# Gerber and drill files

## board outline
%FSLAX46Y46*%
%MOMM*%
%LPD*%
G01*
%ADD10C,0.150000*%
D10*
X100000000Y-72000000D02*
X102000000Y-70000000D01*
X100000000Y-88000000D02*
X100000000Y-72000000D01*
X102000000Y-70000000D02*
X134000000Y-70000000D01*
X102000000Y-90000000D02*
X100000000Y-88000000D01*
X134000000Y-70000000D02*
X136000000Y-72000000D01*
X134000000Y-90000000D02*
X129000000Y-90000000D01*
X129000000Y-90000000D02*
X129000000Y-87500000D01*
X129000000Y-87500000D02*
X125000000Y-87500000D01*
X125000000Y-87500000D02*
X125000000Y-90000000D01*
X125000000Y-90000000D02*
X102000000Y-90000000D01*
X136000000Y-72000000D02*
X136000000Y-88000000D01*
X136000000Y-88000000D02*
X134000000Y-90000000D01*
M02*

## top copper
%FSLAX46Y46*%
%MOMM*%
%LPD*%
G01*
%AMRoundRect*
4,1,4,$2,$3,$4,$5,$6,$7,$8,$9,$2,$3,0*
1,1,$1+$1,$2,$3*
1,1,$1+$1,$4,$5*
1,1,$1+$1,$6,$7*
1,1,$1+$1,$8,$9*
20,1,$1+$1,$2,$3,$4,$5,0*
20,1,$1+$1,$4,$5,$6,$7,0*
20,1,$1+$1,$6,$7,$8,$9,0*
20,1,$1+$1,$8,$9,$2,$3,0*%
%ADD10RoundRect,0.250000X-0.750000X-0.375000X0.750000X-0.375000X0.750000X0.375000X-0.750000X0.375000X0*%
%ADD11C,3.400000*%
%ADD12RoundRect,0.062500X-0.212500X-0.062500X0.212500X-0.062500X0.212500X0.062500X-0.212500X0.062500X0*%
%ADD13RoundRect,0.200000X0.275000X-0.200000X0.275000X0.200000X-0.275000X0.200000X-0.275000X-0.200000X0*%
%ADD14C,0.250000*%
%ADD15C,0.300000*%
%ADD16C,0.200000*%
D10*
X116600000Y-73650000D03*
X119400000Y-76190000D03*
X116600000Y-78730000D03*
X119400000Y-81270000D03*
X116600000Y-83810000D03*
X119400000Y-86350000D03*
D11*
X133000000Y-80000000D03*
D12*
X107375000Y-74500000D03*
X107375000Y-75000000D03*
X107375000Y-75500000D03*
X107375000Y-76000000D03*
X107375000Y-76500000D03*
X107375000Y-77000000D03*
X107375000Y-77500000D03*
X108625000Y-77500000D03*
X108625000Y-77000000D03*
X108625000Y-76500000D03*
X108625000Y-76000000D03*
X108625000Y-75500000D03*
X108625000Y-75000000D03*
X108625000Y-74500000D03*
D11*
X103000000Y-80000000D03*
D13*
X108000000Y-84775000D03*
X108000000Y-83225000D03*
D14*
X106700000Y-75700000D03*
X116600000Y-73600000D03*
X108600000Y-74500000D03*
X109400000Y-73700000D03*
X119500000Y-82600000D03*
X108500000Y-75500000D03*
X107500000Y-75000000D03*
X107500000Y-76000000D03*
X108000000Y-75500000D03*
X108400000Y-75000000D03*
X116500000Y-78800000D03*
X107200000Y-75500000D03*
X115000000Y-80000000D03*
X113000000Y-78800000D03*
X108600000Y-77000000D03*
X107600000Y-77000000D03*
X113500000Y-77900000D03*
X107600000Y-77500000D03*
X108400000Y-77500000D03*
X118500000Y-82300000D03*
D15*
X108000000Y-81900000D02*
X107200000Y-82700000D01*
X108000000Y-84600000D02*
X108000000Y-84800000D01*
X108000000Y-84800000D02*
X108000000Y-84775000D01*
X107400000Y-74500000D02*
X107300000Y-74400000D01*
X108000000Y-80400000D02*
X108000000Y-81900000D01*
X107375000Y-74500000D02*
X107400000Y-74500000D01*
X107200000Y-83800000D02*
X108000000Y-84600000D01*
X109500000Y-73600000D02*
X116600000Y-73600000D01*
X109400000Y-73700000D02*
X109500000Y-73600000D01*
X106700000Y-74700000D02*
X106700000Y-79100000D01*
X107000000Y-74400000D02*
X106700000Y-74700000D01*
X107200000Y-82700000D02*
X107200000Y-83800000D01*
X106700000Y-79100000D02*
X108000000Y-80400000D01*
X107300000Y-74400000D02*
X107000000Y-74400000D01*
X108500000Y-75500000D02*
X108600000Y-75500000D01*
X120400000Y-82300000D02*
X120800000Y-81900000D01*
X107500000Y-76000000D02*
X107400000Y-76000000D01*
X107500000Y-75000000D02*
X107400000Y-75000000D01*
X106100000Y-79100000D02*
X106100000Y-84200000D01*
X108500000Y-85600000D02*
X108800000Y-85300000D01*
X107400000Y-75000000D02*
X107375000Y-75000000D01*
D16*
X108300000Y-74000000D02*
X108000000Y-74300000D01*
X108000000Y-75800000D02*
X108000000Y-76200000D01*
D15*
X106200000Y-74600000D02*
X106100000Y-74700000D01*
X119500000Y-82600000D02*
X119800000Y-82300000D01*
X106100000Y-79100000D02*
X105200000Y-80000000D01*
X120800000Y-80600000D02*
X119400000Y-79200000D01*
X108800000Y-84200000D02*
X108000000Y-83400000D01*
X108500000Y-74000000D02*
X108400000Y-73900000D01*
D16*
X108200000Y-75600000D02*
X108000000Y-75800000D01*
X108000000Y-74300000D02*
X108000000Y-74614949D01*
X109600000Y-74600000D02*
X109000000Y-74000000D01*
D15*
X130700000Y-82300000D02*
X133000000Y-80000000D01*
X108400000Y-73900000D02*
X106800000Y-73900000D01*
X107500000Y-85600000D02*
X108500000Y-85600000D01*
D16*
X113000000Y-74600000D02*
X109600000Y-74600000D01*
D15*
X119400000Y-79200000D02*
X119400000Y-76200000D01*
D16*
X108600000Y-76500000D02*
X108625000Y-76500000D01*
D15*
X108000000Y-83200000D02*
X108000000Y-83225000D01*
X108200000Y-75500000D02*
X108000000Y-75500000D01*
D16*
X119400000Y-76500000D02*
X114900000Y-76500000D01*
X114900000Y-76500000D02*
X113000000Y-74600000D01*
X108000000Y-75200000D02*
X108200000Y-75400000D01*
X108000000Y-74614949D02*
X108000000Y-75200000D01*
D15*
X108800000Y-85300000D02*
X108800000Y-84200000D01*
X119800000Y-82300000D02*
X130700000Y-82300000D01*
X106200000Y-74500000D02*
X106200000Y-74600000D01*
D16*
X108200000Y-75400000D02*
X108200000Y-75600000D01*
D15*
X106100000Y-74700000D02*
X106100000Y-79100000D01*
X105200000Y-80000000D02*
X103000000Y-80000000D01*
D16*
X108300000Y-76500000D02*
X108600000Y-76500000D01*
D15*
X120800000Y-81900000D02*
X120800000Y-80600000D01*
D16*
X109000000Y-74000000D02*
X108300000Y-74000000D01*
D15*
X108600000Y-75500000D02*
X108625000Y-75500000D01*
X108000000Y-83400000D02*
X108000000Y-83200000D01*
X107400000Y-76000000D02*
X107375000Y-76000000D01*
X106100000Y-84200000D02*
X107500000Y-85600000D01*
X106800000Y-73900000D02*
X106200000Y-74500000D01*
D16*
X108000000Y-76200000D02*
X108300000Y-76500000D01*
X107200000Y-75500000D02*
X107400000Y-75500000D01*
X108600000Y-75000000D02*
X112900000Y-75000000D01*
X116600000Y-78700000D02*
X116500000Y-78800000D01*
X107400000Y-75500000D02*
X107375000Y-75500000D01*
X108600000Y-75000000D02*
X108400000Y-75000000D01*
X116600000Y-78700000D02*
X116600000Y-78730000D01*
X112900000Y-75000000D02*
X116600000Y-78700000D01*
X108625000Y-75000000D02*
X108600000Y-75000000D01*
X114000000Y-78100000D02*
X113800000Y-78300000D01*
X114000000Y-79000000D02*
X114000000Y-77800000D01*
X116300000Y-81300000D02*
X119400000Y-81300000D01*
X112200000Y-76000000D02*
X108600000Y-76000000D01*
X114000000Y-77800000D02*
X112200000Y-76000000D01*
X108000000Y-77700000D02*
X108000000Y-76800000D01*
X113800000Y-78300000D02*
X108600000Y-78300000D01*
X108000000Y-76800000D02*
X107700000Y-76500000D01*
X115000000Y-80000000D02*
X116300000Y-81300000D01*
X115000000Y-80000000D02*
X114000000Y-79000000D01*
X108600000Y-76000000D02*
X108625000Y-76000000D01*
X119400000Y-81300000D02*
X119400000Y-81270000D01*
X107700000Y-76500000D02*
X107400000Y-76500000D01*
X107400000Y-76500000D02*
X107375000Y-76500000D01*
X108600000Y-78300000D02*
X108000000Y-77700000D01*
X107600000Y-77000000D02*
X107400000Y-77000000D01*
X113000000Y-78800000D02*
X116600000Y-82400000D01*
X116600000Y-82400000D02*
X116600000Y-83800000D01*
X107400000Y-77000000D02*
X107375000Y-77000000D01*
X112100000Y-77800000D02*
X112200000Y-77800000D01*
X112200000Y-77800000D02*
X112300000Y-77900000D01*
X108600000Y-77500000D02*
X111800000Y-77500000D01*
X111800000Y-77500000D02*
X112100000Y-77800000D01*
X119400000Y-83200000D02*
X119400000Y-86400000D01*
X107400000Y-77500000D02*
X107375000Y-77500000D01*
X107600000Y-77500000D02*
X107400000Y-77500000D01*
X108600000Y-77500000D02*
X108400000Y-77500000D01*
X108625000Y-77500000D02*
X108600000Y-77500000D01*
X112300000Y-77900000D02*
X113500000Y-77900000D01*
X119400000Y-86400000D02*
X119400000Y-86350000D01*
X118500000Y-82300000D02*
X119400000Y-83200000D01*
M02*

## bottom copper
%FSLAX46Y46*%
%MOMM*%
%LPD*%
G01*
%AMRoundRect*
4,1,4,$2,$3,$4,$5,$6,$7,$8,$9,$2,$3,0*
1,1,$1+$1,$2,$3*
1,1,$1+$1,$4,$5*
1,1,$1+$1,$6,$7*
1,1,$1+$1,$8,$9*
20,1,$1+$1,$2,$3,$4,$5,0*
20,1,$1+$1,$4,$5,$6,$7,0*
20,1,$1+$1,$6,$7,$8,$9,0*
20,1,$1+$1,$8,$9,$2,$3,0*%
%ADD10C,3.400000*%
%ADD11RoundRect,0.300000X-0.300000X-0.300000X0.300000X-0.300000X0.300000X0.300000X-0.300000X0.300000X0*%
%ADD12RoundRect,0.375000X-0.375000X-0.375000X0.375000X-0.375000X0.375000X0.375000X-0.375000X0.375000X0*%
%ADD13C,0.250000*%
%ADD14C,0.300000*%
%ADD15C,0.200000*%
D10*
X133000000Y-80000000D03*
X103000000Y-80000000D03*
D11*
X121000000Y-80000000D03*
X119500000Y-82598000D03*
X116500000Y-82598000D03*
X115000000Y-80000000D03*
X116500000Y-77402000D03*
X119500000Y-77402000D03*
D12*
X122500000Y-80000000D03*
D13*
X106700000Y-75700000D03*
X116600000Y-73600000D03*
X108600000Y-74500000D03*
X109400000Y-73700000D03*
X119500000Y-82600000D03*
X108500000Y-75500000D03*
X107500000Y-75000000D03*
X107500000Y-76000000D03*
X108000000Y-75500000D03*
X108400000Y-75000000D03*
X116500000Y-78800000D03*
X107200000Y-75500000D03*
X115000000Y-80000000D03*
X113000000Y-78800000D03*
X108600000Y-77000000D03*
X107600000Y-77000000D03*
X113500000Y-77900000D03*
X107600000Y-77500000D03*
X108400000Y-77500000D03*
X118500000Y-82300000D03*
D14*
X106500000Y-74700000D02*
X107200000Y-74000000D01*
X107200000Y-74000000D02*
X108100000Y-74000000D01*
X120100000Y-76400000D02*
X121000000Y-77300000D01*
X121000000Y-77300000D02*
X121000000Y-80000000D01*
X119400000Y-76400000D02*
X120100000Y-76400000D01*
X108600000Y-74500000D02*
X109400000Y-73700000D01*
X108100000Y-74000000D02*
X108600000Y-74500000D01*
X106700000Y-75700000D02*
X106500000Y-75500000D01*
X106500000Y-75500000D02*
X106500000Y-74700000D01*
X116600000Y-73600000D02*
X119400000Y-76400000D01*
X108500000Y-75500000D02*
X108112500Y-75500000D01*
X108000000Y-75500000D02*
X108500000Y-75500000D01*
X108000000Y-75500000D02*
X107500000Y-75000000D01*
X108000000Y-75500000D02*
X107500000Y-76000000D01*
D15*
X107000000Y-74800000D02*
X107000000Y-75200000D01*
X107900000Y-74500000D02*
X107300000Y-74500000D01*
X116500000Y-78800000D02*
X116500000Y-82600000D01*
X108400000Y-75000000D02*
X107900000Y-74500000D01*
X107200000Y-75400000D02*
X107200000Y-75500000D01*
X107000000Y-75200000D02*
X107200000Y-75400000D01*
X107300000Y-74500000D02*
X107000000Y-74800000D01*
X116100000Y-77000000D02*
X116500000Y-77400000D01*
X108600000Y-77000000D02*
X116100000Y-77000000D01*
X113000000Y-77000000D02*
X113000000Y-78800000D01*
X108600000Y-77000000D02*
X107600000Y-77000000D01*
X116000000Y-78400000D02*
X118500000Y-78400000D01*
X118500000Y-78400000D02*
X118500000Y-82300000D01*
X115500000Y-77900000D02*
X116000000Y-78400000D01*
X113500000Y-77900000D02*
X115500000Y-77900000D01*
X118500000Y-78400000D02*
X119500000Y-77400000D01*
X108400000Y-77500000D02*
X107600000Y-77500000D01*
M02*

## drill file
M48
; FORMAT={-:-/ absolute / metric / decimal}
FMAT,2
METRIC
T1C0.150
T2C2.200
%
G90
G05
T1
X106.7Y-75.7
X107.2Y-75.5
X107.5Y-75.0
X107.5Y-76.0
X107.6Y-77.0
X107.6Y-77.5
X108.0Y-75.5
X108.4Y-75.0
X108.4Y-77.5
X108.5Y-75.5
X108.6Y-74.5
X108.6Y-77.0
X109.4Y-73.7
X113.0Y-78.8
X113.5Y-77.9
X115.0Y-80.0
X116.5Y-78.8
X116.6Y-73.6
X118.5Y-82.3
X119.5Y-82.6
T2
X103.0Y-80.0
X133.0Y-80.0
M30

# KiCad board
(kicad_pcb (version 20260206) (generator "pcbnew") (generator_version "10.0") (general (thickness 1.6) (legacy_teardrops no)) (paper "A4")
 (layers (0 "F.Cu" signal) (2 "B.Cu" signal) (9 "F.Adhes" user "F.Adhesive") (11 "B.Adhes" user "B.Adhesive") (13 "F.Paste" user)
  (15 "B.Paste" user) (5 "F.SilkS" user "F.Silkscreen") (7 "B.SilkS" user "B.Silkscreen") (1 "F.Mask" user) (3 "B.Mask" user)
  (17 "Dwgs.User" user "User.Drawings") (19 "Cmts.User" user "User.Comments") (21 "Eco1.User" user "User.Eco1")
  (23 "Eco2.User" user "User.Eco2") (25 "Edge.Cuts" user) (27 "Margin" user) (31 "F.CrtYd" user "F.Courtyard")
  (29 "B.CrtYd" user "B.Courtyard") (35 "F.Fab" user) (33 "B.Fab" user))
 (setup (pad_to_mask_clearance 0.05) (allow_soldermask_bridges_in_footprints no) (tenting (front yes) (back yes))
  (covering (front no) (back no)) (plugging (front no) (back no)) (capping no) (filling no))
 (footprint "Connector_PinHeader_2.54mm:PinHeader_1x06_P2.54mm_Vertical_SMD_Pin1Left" (layer "F.Cu") (at 118 73.65)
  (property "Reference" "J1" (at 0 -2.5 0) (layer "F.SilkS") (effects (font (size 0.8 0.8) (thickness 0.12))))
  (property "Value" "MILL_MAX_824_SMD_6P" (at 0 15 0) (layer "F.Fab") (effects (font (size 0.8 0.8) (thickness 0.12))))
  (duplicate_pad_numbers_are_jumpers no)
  (pad "1" smd roundrect (at -1.4 0) (size 2 1.25) (layers "F.Cu" "F.Mask" "F.Paste") (roundrect_rratio 0.2) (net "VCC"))
  (pad "2" smd roundrect (at 1.4 2.54) (size 2 1.25) (layers "F.Cu" "F.Mask" "F.Paste") (roundrect_rratio 0.2) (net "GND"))
  (pad "3" smd roundrect (at -1.4 5.08) (size 2 1.25) (layers "F.Cu" "F.Mask" "F.Paste") (roundrect_rratio 0.2) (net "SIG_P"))
  (pad "4" smd roundrect (at 1.4 7.62) (size 2 1.25) (layers "F.Cu" "F.Mask" "F.Paste") (roundrect_rratio 0.2) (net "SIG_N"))
  (pad "5" smd roundrect (at -1.4 10.16) (size 2 1.25) (layers "F.Cu" "F.Mask" "F.Paste") (roundrect_rratio 0.2) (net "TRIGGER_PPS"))
  (pad "6" smd roundrect (at 1.4 12.7) (size 2 1.25) (layers "F.Cu" "F.Mask" "F.Paste") (roundrect_rratio 0.2) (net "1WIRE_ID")))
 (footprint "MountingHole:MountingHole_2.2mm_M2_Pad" (layer "F.Cu") (at 133 80)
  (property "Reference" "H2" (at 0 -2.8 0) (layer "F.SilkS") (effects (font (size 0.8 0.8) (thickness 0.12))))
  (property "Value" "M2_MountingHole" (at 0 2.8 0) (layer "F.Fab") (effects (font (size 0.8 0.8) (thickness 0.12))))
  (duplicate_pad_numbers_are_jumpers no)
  (pad "1" thru_hole circle (at 0 0) (size 3.4 3.4) (drill 2.2) (layers "*.Cu" "*.Mask") (remove_unused_layers no) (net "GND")))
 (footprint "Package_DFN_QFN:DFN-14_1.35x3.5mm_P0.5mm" (layer "F.Cu") (at 108 76)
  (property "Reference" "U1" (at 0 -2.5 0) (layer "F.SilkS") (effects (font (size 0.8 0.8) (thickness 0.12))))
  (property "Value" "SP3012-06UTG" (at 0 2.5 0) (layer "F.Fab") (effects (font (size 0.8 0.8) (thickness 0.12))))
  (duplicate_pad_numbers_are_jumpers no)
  (pad "1" smd roundrect (at -0.625 -1.5) (size 0.55 0.25) (layers "F.Cu" "F.Mask" "F.Paste") (roundrect_rratio 0.25) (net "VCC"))
  (pad "2" smd roundrect (at -0.625 -1) (size 0.55 0.25) (layers "F.Cu" "F.Mask" "F.Paste") (roundrect_rratio 0.25) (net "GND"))
  (pad "3" smd roundrect (at -0.625 -0.5) (size 0.55 0.25) (layers "F.Cu" "F.Mask" "F.Paste") (roundrect_rratio 0.25) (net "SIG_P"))
  (pad "4" smd roundrect (at -0.625 0) (size 0.55 0.25) (layers "F.Cu" "F.Mask" "F.Paste") (roundrect_rratio 0.25) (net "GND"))
  (pad "5" smd roundrect (at -0.625 0.5) (size 0.55 0.25) (layers "F.Cu" "F.Mask" "F.Paste") (roundrect_rratio 0.25) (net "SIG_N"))
  (pad "6" smd roundrect (at -0.625 1) (size 0.55 0.25) (layers "F.Cu" "F.Mask" "F.Paste") (roundrect_rratio 0.25) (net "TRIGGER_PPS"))
  (pad "7" smd roundrect (at -0.625 1.5) (size 0.55 0.25) (layers "F.Cu" "F.Mask" "F.Paste") (roundrect_rratio 0.25) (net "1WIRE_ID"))
  (pad "8" smd roundrect (at 0.625 1.5) (size 0.55 0.25) (layers "F.Cu" "F.Mask" "F.Paste") (roundrect_rratio 0.25) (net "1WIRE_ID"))
  (pad "9" smd roundrect (at 0.625 1) (size 0.55 0.25) (layers "F.Cu" "F.Mask" "F.Paste") (roundrect_rratio 0.25) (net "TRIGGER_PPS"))
  (pad "10" smd roundrect (at 0.625 0.5) (size 0.55 0.25) (layers "F.Cu" "F.Mask" "F.Paste") (roundrect_rratio 0.25) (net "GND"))
  (pad "11" smd roundrect (at 0.625 0) (size 0.55 0.25) (layers "F.Cu" "F.Mask" "F.Paste") (roundrect_rratio 0.25) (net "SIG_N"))
  (pad "12" smd roundrect (at 0.625 -0.5) (size 0.55 0.25) (layers "F.Cu" "F.Mask" "F.Paste") (roundrect_rratio 0.25) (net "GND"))
  (pad "13" smd roundrect (at 0.625 -1) (size 0.55 0.25) (layers "F.Cu" "F.Mask" "F.Paste") (roundrect_rratio 0.25) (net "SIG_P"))
  (pad "14" smd roundrect (at 0.625 -1.5) (size 0.55 0.25) (layers "F.Cu" "F.Mask" "F.Paste") (roundrect_rratio 0.25) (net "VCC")))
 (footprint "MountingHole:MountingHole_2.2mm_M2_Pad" (layer "F.Cu") (at 103 80)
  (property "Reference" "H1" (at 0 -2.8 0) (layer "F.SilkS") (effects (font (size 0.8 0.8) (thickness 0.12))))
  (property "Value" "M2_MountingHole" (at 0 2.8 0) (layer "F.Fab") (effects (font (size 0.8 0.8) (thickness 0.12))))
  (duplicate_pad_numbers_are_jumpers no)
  (pad "1" thru_hole circle (at 0 0) (size 3.4 3.4) (drill 2.2) (layers "*.Cu" "*.Mask") (remove_unused_layers no) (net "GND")))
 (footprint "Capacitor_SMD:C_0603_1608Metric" (layer "F.Cu") (at 108 84 90)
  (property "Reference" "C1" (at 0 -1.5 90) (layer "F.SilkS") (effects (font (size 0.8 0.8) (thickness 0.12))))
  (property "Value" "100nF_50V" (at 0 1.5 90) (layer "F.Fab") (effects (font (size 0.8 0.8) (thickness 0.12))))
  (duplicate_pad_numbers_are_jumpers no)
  (pad "1" smd roundrect (at -0.775 0 90) (size 0.8 0.95) (layers "F.Cu" "F.Mask" "F.Paste") (roundrect_rratio 0.25) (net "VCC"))
  (pad "2" smd roundrect (at 0.775 0 90) (size 0.8 0.95) (layers "F.Cu" "F.Mask" "F.Paste") (roundrect_rratio 0.25) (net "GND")))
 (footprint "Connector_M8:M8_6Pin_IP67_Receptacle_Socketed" (layer "B.Cu") (at 118 80)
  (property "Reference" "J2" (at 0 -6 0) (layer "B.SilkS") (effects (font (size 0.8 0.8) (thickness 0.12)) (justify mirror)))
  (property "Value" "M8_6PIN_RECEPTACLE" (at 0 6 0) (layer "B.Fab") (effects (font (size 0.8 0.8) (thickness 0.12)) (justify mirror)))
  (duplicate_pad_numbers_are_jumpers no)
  (pad "1" smd roundrect (at 3 0) (size 1.2 1.2) (layers "B.Cu" "B.Mask" "B.Paste") (roundrect_rratio 0.25) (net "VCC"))
  (pad "2" smd roundrect (at 1.5 2.598) (size 1.2 1.2) (layers "B.Cu" "B.Mask" "B.Paste") (roundrect_rratio 0.25) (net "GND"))
  (pad "3" smd roundrect (at -1.5 2.598) (size 1.2 1.2) (layers "B.Cu" "B.Mask" "B.Paste") (roundrect_rratio 0.25) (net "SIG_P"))
  (pad "4" smd roundrect (at -3 0) (size 1.2 1.2) (layers "B.Cu" "B.Mask" "B.Paste") (roundrect_rratio 0.25) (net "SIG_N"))
  (pad "5" smd roundrect (at -1.5 -2.598) (size 1.2 1.2) (layers "B.Cu" "B.Mask" "B.Paste") (roundrect_rratio 0.25) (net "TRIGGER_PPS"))
  (pad "6" smd roundrect (at 1.5 -2.598) (size 1.2 1.2) (layers "B.Cu" "B.Mask" "B.Paste") (roundrect_rratio 0.25) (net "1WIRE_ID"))
  (pad "7" smd roundrect (at 4.5 0) (size 1.5 1.5) (layers "B.Cu" "B.Mask" "B.Paste") (roundrect_rratio 0.25) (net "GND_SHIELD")))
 (gr_line (start 100 72) (end 102 70) (stroke (width 0.15) (type solid)) (layer "Edge.Cuts"))
 (gr_line (start 100 88) (end 100 72) (stroke (width 0.15) (type solid)) (layer "Edge.Cuts"))
 (gr_line (start 102 70) (end 134 70) (stroke (width 0.15) (type solid)) (layer "Edge.Cuts"))
 (gr_line (start 102 90) (end 100 88) (stroke (width 0.15) (type solid)) (layer "Edge.Cuts"))
 (gr_line (start 134 70) (end 136 72) (stroke (width 0.15) (type solid)) (layer "Edge.Cuts"))
 (gr_line (start 134 90) (end 129 90) (stroke (width 0.15) (type solid)) (layer "Edge.Cuts"))
 (gr_line (start 129 90) (end 129 87.5) (stroke (width 0.15) (type solid)) (layer "Edge.Cuts"))
 (gr_line (start 129 87.5) (end 125 87.5) (stroke (width 0.15) (type solid)) (layer "Edge.Cuts"))
 (gr_line (start 125 87.5) (end 125 90) (stroke (width 0.15) (type solid)) (layer "Edge.Cuts"))
 (gr_line (start 125 90) (end 102 90) (stroke (width 0.15) (type solid)) (layer "Edge.Cuts"))
 (gr_line (start 136 72) (end 136 88) (stroke (width 0.15) (type solid)) (layer "Edge.Cuts"))
 (gr_line (start 136 88) (end 134 90) (stroke (width 0.15) (type solid)) (layer "Edge.Cuts"))
 (segment (start 108 81.9) (end 107.2 82.7) (width 0.3) (layer "F.Cu") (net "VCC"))
 (segment (start 108 84.6) (end 108 84.8) (width 0.3) (layer "F.Cu") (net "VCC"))
 (segment (start 108 84.8) (end 108 84.775) (width 0.3) (layer "F.Cu") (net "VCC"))
 (segment (start 107.4 74.5) (end 107.3 74.4) (width 0.3) (layer "F.Cu") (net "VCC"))
 (segment (start 108 80.4) (end 108 81.9) (width 0.3) (layer "F.Cu") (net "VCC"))
 (segment (start 107.375 74.5) (end 107.4 74.5) (width 0.3) (layer "F.Cu") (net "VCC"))
 (segment (start 107.2 83.8) (end 108 84.6) (width 0.3) (layer "F.Cu") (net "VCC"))
 (segment (start 109.5 73.6) (end 116.6 73.6) (width 0.3) (layer "F.Cu") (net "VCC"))
 (segment (start 109.4 73.7) (end 109.5 73.6) (width 0.3) (layer "F.Cu") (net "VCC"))
 (segment (start 106.7 74.7) (end 106.7 79.1) (width 0.3) (layer "F.Cu") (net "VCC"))
 (segment (start 107 74.4) (end 106.7 74.7) (width 0.3) (layer "F.Cu") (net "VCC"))
 (segment (start 107.2 82.7) (end 107.2 83.8) (width 0.3) (layer "F.Cu") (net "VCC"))
 (segment (start 106.7 79.1) (end 108 80.4) (width 0.3) (layer "F.Cu") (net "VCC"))
 (segment (start 107.3 74.4) (end 107 74.4) (width 0.3) (layer "F.Cu") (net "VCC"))
 (via (at 106.7 75.7) (size 0.25) (drill 0.15) (layers "F.Cu" "B.Cu") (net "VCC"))
 (via (at 116.6 73.6) (size 0.25) (drill 0.15) (layers "F.Cu" "B.Cu") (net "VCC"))
 (via (at 108.6 74.5) (size 0.25) (drill 0.15) (layers "F.Cu" "B.Cu") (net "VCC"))
 (via (at 109.4 73.7) (size 0.25) (drill 0.15) (layers "F.Cu" "B.Cu") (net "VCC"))
 (segment (start 106.5 74.7) (end 107.2 74) (width 0.3) (layer "B.Cu") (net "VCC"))
 (segment (start 107.2 74) (end 108.1 74) (width 0.3) (layer "B.Cu") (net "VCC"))
 (segment (start 120.1 76.4) (end 121 77.3) (width 0.3) (layer "B.Cu") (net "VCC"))
 (segment (start 121 77.3) (end 121 80) (width 0.3) (layer "B.Cu") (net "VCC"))
 (segment (start 119.4 76.4) (end 120.1 76.4) (width 0.3) (layer "B.Cu") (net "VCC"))
 (segment (start 108.6 74.5) (end 109.4 73.7) (width 0.3) (layer "B.Cu") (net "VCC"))
 (segment (start 108.1 74) (end 108.6 74.5) (width 0.3) (layer "B.Cu") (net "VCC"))
 (segment (start 106.7 75.7) (end 106.5 75.5) (width 0.3) (layer "B.Cu") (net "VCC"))
 (segment (start 106.5 75.5) (end 106.5 74.7) (width 0.3) (layer "B.Cu") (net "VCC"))
 (segment (start 116.6 73.6) (end 119.4 76.4) (width 0.3) (layer "B.Cu") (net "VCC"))
 (segment (start 108.5 75.5) (end 108.6 75.5) (width 0.3) (layer "F.Cu") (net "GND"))
 (segment (start 120.4 82.3) (end 120.8 81.9) (width 0.3) (layer "F.Cu") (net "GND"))
 (segment (start 107.5 76) (end 107.4 76) (width 0.3) (layer "F.Cu") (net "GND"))
 (segment (start 107.5 75) (end 107.4 75) (width 0.3) (layer "F.Cu") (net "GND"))
 (segment (start 106.1 79.1) (end 106.1 84.2) (width 0.3) (layer "F.Cu") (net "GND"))
 (segment (start 108.5 85.6) (end 108.8 85.3) (width 0.3) (layer "F.Cu") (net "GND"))
 (segment (start 107.4 75) (end 107.375 75) (width 0.3) (layer "F.Cu") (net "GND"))
 (segment (start 108.3 74) (end 108 74.3) (width 0.2) (layer "F.Cu") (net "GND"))
 (segment (start 108 75.8) (end 108 76.2) (width 0.2) (layer "F.Cu") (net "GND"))
 (segment (start 106.2 74.6) (end 106.1 74.7) (width 0.3) (layer "F.Cu") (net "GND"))
 (segment (start 119.5 82.6) (end 119.8 82.3) (width 0.3) (layer "F.Cu") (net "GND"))
 (segment (start 106.1 79.1) (end 105.2 80) (width 0.3) (layer "F.Cu") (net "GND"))
 (segment (start 120.8 80.6) (end 119.4 79.2) (width 0.3) (layer "F.Cu") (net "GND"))
 (segment (start 108.8 84.2) (end 108 83.4) (width 0.3) (layer "F.Cu") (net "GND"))
 (segment (start 108.5 74) (end 108.4 73.9) (width 0.3) (layer "F.Cu") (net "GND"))
 (segment (start 108.2 75.6) (end 108 75.8) (width 0.2) (layer "F.Cu") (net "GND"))
 (segment (start 108 74.3) (end 108 74.614949) (width 0.2) (layer "F.Cu") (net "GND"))
 (segment (start 109.6 74.6) (end 109 74) (width 0.2) (layer "F.Cu") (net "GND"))
 (segment (start 130.7 82.3) (end 133 80) (width 0.3) (layer "F.Cu") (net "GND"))
 (segment (start 108.4 73.9) (end 106.8 73.9) (width 0.3) (layer "F.Cu") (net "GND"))
 (segment (start 107.5 85.6) (end 108.5 85.6) (width 0.3) (layer "F.Cu") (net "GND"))
 (segment (start 113 74.6) (end 109.6 74.6) (width 0.2) (layer "F.Cu") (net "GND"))
 (segment (start 119.4 79.2) (end 119.4 76.2) (width 0.3) (layer "F.Cu") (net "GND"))
 (segment (start 108.6 76.5) (end 108.625 76.5) (width 0.2) (layer "F.Cu") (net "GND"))
 (segment (start 108 83.2) (end 108 83.225) (width 0.3) (layer "F.Cu") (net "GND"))
 (segment (start 108.2 75.5) (end 108 75.5) (width 0.3) (layer "F.Cu") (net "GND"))
 (segment (start 119.4 76.5) (end 114.9 76.5) (width 0.2) (layer "F.Cu") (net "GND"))
 (segment (start 114.9 76.5) (end 113 74.6) (width 0.2) (layer "F.Cu") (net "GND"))
 (segment (start 108 75.2) (end 108.2 75.4) (width 0.2) (layer "F.Cu") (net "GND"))
 (segment (start 108 74.614949) (end 108 75.2) (width 0.2) (layer "F.Cu") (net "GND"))
 (segment (start 108.8 85.3) (end 108.8 84.2) (width 0.3) (layer "F.Cu") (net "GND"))
 (segment (start 119.8 82.3) (end 130.7 82.3) (width 0.3) (layer "F.Cu") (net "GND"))
 (segment (start 106.2 74.5) (end 106.2 74.6) (width 0.3) (layer "F.Cu") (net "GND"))
 (segment (start 108.2 75.4) (end 108.2 75.6) (width 0.2) (layer "F.Cu") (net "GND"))
 (segment (start 106.1 74.7) (end 106.1 79.1) (width 0.3) (layer "F.Cu") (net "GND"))
 (segment (start 105.2 80) (end 103 80) (width 0.3) (layer "F.Cu") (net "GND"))
 (segment (start 108.3 76.5) (end 108.6 76.5) (width 0.2) (layer "F.Cu") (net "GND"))
 (segment (start 120.8 81.9) (end 120.8 80.6) (width 0.3) (layer "F.Cu") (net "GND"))
 (segment (start 109 74) (end 108.3 74) (width 0.2) (layer "F.Cu") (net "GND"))
 (segment (start 108.6 75.5) (end 108.625 75.5) (width 0.3) (layer "F.Cu") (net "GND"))
 (segment (start 108 83.4) (end 108 83.2) (width 0.3) (layer "F.Cu") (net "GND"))
 (segment (start 107.4 76) (end 107.375 76) (width 0.3) (layer "F.Cu") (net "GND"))
 (segment (start 106.1 84.2) (end 107.5 85.6) (width 0.3) (layer "F.Cu") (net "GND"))
 (segment (start 106.8 73.9) (end 106.2 74.5) (width 0.3) (layer "F.Cu") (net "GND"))
 (segment (start 108 76.2) (end 108.3 76.5) (width 0.2) (layer "F.Cu") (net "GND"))
 (via (at 119.5 82.6) (size 0.25) (drill 0.15) (layers "F.Cu" "B.Cu") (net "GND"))
 (via (at 108.5 75.5) (size 0.25) (drill 0.15) (layers "F.Cu" "B.Cu") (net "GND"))
 (via (at 107.5 75) (size 0.25) (drill 0.15) (layers "F.Cu" "B.Cu") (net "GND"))
 (via (at 107.5 76) (size 0.25) (drill 0.15) (layers "F.Cu" "B.Cu") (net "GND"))
 (via (at 108 75.5) (size 0.25) (drill 0.15) (layers "F.Cu" "B.Cu") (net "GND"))
 (segment (start 108.5 75.5) (end 108.1125 75.5) (width 0.3) (layer "B.Cu") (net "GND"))
 (segment (start 108 75.5) (end 108.5 75.5) (width 0.3) (layer "B.Cu") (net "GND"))
 (segment (start 108 75.5) (end 107.5 75) (width 0.3) (layer "B.Cu") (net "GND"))
 (segment (start 108 75.5) (end 107.5 76) (width 0.3) (layer "B.Cu") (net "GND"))
 (segment (start 107.2 75.5) (end 107.4 75.5) (width 0.2) (layer "F.Cu") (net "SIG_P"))
 (segment (start 108.6 75) (end 112.9 75) (width 0.2) (layer "F.Cu") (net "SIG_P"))
 (segment (start 116.6 78.7) (end 116.5 78.8) (width 0.2) (layer "F.Cu") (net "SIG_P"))
 (segment (start 107.4 75.5) (end 107.375 75.5) (width 0.2) (layer "F.Cu") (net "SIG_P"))
 (segment (start 108.6 75) (end 108.4 75) (width 0.2) (layer "F.Cu") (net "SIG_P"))
 (segment (start 116.6 78.7) (end 116.6 78.73) (width 0.2) (layer "F.Cu") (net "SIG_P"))
 (segment (start 112.9 75) (end 116.6 78.7) (width 0.2) (layer "F.Cu") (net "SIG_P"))
 (segment (start 108.625 75) (end 108.6 75) (width 0.2) (layer "F.Cu") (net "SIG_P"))
 (via (at 108.4 75) (size 0.25) (drill 0.15) (layers "F.Cu" "B.Cu") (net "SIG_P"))
 (via (at 116.5 78.8) (size 0.25) (drill 0.15) (layers "F.Cu" "B.Cu") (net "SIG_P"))
 (via (at 107.2 75.5) (size 0.25) (drill 0.15) (layers "F.Cu" "B.Cu") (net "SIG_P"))
 (segment (start 107 74.8) (end 107 75.2) (width 0.2) (layer "B.Cu") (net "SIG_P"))
 (segment (start 107.9 74.5) (end 107.3 74.5) (width 0.2) (layer "B.Cu") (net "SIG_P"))
 (segment (start 116.5 78.8) (end 116.5 82.6) (width 0.2) (layer "B.Cu") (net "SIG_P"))
 (segment (start 108.4 75) (end 107.9 74.5) (width 0.2) (layer "B.Cu") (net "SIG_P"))
 (segment (start 107.2 75.4) (end 107.2 75.5) (width 0.2) (layer "B.Cu") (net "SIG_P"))
 (segment (start 107 75.2) (end 107.2 75.4) (width 0.2) (layer "B.Cu") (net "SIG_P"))
 (segment (start 107.3 74.5) (end 107 74.8) (width 0.2) (layer "B.Cu") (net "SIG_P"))
 (segment (start 114 78.1) (end 113.8 78.3) (width 0.2) (layer "F.Cu") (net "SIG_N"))
 (segment (start 114 79) (end 114 77.8) (width 0.2) (layer "F.Cu") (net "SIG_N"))
 (segment (start 116.3 81.3) (end 119.4 81.3) (width 0.2) (layer "F.Cu") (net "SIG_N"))
 (segment (start 112.2 76) (end 108.6 76) (width 0.2) (layer "F.Cu") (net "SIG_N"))
 (segment (start 114 77.8) (end 112.2 76) (width 0.2) (layer "F.Cu") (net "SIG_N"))
 (segment (start 108 77.7) (end 108 76.8) (width 0.2) (layer "F.Cu") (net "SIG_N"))
 (segment (start 113.8 78.3) (end 108.6 78.3) (width 0.2) (layer "F.Cu") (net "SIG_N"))
 (segment (start 108 76.8) (end 107.7 76.5) (width 0.2) (layer "F.Cu") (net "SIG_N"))
 (segment (start 115 80) (end 116.3 81.3) (width 0.2) (layer "F.Cu") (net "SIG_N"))
 (segment (start 115 80) (end 114 79) (width 0.2) (layer "F.Cu") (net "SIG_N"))
 (segment (start 108.6 76) (end 108.625 76) (width 0.2) (layer "F.Cu") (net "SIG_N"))
 (segment (start 119.4 81.3) (end 119.4 81.27) (width 0.2) (layer "F.Cu") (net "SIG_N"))
 (segment (start 107.7 76.5) (end 107.4 76.5) (width 0.2) (layer "F.Cu") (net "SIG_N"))
 (segment (start 107.4 76.5) (end 107.375 76.5) (width 0.2) (layer "F.Cu") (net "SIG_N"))
 (segment (start 108.6 78.3) (end 108 77.7) (width 0.2) (layer "F.Cu") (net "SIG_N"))
 (via (at 115 80) (size 0.25) (drill 0.15) (layers "F.Cu" "B.Cu") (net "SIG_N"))
 (segment (start 107.6 77) (end 107.4 77) (width 0.2) (layer "F.Cu") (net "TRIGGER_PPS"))
 (segment (start 113 78.8) (end 116.6 82.4) (width 0.2) (layer "F.Cu") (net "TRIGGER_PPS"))
 (segment (start 116.6 82.4) (end 116.6 83.8) (width 0.2) (layer "F.Cu") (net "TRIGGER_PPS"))
 (segment (start 107.4 77) (end 107.375 77) (width 0.2) (layer "F.Cu") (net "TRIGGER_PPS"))
 (via (at 113 78.8) (size 0.25) (drill 0.15) (layers "F.Cu" "B.Cu") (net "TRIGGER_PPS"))
 (via (at 108.6 77) (size 0.25) (drill 0.15) (layers "F.Cu" "B.Cu") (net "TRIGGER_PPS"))
 (via (at 107.6 77) (size 0.25) (drill 0.15) (layers "F.Cu" "B.Cu") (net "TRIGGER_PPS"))
 (segment (start 116.1 77) (end 116.5 77.4) (width 0.2) (layer "B.Cu") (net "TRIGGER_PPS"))
 (segment (start 108.6 77) (end 116.1 77) (width 0.2) (layer "B.Cu") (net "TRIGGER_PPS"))
 (segment (start 113 77) (end 113 78.8) (width 0.2) (layer "B.Cu") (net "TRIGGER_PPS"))
 (segment (start 108.6 77) (end 107.6 77) (width 0.2) (layer "B.Cu") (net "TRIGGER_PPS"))
 (segment (start 112.1 77.8) (end 112.2 77.8) (width 0.2) (layer "F.Cu") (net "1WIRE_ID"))
 (segment (start 112.2 77.8) (end 112.3 77.9) (width 0.2) (layer "F.Cu") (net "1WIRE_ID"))
 (segment (start 108.6 77.5) (end 111.8 77.5) (width 0.2) (layer "F.Cu") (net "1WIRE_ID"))
 (segment (start 111.8 77.5) (end 112.1 77.8) (width 0.2) (layer "F.Cu") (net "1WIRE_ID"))
 (segment (start 119.4 83.2) (end 119.4 86.4) (width 0.2) (layer "F.Cu") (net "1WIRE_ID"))
 (segment (start 107.4 77.5) (end 107.375 77.5) (width 0.2) (layer "F.Cu") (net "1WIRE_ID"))
 (segment (start 107.6 77.5) (end 107.4 77.5) (width 0.2) (layer "F.Cu") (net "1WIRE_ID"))
 (segment (start 108.6 77.5) (end 108.4 77.5) (width 0.2) (layer "F.Cu") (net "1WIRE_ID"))
 (segment (start 108.625 77.5) (end 108.6 77.5) (width 0.2) (layer "F.Cu") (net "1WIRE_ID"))
 (segment (start 112.3 77.9) (end 113.5 77.9) (width 0.2) (layer "F.Cu") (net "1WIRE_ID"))
 (segment (start 119.4 86.4) (end 119.4 86.35) (width 0.2) (layer "F.Cu") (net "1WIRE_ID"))
 (segment (start 118.5 82.3) (end 119.4 83.2) (width 0.2) (layer "F.Cu") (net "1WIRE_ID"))
 (via (at 113.5 77.9) (size 0.25) (drill 0.15) (layers "F.Cu" "B.Cu") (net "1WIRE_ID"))
 (via (at 107.6 77.5) (size 0.25) (drill 0.15) (layers "F.Cu" "B.Cu") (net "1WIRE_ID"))
 (via (at 108.4 77.5) (size 0.25) (drill 0.15) (layers "F.Cu" "B.Cu") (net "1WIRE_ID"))
 (via (at 118.5 82.3) (size 0.25) (drill 0.15) (layers "F.Cu" "B.Cu") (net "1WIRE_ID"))
 (segment (start 116 78.4) (end 118.5 78.4) (width 0.2) (layer "B.Cu") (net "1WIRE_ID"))
 (segment (start 118.5 78.4) (end 118.5 82.3) (width 0.2) (layer "B.Cu") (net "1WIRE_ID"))
 (segment (start 115.5 77.9) (end 116 78.4) (width 0.2) (layer "B.Cu") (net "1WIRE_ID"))
 (segment (start 113.5 77.9) (end 115.5 77.9) (width 0.2) (layer "B.Cu") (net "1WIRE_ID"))
 (segment (start 118.5 78.4) (end 119.5 77.4) (width 0.2) (layer "B.Cu") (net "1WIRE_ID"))
 (segment (start 108.4 77.5) (end 107.6 77.5) (width 0.2) (layer "B.Cu") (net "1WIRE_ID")))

